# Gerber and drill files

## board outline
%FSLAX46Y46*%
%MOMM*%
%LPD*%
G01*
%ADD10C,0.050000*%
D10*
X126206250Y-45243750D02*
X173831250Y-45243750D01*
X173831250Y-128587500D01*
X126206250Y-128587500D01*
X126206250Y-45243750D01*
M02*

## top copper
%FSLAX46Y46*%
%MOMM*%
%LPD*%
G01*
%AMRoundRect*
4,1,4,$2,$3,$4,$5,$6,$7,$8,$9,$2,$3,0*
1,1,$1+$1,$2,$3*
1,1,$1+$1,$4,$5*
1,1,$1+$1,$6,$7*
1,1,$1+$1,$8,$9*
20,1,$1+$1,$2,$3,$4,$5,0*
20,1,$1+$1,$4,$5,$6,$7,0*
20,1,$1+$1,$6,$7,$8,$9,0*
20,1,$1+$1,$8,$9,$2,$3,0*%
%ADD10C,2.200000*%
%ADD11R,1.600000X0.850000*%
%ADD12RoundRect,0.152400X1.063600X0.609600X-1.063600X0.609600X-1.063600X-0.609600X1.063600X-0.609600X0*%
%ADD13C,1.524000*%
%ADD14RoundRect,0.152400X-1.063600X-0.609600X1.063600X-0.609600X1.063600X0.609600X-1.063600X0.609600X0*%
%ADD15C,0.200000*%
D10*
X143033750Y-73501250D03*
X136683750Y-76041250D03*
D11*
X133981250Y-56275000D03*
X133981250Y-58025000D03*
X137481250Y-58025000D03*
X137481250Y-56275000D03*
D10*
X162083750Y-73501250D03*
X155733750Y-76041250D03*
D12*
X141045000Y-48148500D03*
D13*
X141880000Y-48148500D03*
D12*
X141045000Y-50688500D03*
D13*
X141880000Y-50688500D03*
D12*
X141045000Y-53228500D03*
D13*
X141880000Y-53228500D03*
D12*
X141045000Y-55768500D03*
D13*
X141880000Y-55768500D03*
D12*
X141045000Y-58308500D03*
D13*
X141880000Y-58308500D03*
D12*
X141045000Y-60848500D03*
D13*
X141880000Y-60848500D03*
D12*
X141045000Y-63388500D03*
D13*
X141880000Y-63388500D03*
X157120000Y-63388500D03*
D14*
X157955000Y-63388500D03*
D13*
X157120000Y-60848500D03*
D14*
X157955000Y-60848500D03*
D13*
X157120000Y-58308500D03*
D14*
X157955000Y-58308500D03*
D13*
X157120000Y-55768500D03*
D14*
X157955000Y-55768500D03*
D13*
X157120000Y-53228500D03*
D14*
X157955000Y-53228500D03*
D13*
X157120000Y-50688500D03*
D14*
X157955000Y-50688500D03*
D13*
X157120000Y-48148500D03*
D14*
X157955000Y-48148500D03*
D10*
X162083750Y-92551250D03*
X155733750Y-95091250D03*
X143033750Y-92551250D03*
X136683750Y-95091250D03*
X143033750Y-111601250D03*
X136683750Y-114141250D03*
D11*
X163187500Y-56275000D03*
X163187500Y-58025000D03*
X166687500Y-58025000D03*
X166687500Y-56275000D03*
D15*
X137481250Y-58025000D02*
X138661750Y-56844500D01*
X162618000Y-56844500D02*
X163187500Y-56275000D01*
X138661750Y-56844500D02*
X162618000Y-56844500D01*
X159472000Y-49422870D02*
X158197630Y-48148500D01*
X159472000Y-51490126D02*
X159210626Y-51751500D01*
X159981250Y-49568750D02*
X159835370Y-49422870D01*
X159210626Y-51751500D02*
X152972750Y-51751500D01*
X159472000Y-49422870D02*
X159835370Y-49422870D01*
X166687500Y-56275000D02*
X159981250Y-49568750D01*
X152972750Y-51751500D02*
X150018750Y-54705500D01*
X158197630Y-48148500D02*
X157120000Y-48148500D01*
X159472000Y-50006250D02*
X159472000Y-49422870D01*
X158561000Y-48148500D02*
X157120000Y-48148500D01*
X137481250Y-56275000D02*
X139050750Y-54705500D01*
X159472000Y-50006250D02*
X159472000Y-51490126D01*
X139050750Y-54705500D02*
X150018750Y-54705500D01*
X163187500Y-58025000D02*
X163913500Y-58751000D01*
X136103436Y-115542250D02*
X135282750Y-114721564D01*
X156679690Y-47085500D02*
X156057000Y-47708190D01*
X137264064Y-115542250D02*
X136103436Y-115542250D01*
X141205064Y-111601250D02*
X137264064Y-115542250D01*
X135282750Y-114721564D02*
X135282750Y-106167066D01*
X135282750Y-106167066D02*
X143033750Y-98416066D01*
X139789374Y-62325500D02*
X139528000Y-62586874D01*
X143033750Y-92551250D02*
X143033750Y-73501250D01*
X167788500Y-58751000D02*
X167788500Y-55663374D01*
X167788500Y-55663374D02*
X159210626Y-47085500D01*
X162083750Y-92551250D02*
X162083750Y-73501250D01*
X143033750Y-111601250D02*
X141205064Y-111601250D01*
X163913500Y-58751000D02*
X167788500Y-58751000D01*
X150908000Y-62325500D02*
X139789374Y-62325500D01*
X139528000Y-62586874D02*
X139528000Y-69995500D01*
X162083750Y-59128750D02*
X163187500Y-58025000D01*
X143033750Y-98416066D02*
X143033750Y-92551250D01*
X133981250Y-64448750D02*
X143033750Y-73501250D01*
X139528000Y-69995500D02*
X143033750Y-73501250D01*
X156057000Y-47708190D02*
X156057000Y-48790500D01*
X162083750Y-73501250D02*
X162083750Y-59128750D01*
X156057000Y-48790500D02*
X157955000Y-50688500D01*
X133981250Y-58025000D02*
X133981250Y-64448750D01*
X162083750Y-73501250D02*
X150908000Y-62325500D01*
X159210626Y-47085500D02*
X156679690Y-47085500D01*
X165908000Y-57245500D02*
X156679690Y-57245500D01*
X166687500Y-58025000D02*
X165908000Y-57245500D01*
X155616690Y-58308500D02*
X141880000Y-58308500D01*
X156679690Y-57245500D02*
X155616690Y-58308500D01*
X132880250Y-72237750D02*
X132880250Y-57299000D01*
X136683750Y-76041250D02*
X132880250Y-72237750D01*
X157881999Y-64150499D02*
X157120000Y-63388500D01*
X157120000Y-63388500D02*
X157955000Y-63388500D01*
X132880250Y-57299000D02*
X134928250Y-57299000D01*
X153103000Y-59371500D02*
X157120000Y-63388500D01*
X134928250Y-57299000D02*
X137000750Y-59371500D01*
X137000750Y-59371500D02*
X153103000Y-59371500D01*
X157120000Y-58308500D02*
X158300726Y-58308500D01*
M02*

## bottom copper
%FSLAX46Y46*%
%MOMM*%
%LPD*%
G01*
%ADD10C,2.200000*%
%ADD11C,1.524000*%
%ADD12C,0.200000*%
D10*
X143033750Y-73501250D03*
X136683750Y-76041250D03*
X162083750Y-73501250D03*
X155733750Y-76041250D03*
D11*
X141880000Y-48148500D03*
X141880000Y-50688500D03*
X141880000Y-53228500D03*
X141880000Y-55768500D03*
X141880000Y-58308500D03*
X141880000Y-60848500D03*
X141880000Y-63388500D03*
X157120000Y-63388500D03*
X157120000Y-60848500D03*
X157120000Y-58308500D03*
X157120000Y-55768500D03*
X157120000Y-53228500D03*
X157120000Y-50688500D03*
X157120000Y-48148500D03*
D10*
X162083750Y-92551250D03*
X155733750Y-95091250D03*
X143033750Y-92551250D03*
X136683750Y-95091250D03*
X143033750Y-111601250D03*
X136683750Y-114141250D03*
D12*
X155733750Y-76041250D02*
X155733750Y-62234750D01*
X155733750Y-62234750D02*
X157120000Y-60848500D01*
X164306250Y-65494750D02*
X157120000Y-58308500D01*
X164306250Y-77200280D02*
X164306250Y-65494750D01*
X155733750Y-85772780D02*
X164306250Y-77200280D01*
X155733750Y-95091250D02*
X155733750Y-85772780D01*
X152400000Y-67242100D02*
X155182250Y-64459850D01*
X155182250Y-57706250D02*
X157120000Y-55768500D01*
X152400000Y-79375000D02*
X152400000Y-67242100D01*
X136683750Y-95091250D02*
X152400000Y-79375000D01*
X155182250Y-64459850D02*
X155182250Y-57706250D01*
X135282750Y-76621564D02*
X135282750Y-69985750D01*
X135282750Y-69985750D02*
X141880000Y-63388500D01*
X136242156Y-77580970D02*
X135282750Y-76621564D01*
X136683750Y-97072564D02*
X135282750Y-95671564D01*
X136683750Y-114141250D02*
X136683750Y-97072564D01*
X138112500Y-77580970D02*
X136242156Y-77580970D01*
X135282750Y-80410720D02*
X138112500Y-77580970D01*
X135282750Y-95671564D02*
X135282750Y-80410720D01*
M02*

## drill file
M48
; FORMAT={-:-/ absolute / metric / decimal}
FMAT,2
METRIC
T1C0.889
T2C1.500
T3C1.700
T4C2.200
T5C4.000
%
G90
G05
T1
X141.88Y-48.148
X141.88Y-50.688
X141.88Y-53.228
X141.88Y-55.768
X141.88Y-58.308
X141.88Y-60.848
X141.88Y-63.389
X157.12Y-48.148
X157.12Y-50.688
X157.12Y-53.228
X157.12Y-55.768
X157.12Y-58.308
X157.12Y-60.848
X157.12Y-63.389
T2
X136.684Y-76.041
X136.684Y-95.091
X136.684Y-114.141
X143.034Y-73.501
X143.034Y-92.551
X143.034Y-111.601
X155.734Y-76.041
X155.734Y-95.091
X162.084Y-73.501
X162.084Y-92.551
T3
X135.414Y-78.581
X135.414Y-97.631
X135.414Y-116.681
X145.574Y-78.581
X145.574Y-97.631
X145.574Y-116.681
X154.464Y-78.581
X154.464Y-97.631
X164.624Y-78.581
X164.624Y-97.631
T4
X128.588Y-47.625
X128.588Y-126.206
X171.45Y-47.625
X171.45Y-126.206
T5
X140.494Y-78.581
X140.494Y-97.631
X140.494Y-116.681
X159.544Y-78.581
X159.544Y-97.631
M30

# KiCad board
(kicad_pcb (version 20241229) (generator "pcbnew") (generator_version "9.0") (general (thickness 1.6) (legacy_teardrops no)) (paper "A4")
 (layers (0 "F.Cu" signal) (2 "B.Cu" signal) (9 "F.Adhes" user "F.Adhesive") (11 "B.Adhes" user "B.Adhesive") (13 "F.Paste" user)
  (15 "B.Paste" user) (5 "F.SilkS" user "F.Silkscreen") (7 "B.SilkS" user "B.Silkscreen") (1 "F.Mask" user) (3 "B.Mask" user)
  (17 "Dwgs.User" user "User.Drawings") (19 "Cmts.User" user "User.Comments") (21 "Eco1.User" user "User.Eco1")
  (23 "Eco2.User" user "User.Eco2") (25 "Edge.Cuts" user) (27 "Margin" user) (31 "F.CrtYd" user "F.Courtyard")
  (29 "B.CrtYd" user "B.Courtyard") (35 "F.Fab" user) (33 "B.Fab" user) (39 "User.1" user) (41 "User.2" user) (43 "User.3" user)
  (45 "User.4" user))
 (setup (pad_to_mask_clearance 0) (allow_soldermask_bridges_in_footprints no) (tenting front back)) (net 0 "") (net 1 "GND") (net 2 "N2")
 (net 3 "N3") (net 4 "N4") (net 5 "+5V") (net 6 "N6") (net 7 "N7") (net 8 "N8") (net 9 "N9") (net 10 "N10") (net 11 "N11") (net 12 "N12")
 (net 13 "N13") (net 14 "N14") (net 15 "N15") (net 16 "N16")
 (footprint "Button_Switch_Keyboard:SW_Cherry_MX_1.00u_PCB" (layer "F.Cu") (at 143.03375 73.50125)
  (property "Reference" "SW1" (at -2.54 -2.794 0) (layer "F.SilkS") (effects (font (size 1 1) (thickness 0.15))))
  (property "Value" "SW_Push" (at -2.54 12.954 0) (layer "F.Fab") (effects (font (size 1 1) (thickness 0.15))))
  (pad "" np_thru_hole circle (at -7.62 5.08) (size 1.7 1.7) (drill 1.7) (layers "*.Cu" "*.Mask"))
  (pad "" np_thru_hole circle (at -2.54 5.08) (size 4 4) (drill 4) (layers "*.Cu" "*.Mask"))
  (pad "" np_thru_hole circle (at 2.54 5.08) (size 1.7 1.7) (drill 1.7) (layers "*.Cu" "*.Mask"))
  (pad "1" thru_hole circle (at 0 0) (size 2.2 2.2) (drill 1.5) (layers "*.Cu" "*.Mask") (remove_unused_layers no) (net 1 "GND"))
  (pad "2" thru_hole circle (at -6.35 2.54) (size 2.2 2.2) (drill 1.5) (layers "*.Cu" "*.Mask") (remove_unused_layers no) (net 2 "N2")))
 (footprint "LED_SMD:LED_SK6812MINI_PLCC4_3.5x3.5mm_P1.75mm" (layer "F.Cu") (at 135.73125 57.15)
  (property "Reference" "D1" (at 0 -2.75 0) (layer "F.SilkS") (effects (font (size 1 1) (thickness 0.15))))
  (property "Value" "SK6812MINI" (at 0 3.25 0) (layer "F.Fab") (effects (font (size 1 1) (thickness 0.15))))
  (pad "1" smd rect (at -1.75 -0.875) (size 1.6 0.85) (layers "F.Cu" "F.Mask" "F.Paste") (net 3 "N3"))
  (pad "2" smd rect (at -1.75 0.875) (size 1.6 0.85) (layers "F.Cu" "F.Mask" "F.Paste") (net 1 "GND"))
  (pad "3" smd rect (at 1.75 0.875) (size 1.6 0.85) (layers "F.Cu" "F.Mask" "F.Paste") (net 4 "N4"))
  (pad "4" smd rect (at 1.75 -0.875) (size 1.6 0.85) (layers "F.Cu" "F.Mask" "F.Paste") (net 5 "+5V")))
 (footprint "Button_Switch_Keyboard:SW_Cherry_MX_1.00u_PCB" (layer "F.Cu") (at 162.08375 73.50125)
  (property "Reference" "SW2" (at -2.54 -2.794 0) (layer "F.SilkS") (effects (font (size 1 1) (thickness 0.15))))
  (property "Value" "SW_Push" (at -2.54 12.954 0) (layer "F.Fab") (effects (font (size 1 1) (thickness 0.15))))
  (pad "" np_thru_hole circle (at -7.62 5.08) (size 1.7 1.7) (drill 1.7) (layers "*.Cu" "*.Mask"))
  (pad "" np_thru_hole circle (at -2.54 5.08) (size 4 4) (drill 4) (layers "*.Cu" "*.Mask"))
  (pad "" np_thru_hole circle (at 2.54 5.08) (size 1.7 1.7) (drill 1.7) (layers "*.Cu" "*.Mask"))
  (pad "1" thru_hole circle (at 0 0) (size 2.2 2.2) (drill 1.5) (layers "*.Cu" "*.Mask") (remove_unused_layers no) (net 1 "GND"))
  (pad "2" thru_hole circle (at -6.35 2.54) (size 2.2 2.2) (drill 1.5) (layers "*.Cu" "*.Mask") (remove_unused_layers no) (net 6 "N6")))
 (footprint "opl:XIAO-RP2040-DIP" (layer "F.Cu") (at 149.5 55.7685)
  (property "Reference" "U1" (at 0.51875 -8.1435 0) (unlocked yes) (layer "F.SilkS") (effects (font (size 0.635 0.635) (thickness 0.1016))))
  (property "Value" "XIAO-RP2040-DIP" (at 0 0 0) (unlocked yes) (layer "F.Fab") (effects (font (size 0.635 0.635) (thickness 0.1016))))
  (pad "1" smd roundrect (at -8.455 -7.62 180) (size 2.432 1.524) (layers "F.Cu" "F.Mask") (roundrect_rratio 0.1) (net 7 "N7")
   (thermal_bridge_angle 45))
  (pad "1" thru_hole circle (at -7.62 -7.62 180) (size 1.524 1.524) (drill 0.889) (layers "*.Cu" "*.Mask") (remove_unused_layers no)
   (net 7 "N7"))
  (pad "2" smd roundrect (at -8.455 -5.08 180) (size 2.432 1.524) (layers "F.Cu" "F.Mask") (roundrect_rratio 0.1) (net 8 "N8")
   (thermal_bridge_angle 45))
  (pad "2" thru_hole circle (at -7.62 -5.08 180) (size 1.524 1.524) (drill 0.889) (layers "*.Cu" "*.Mask") (remove_unused_layers no)
   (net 8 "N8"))
  (pad "3" smd roundrect (at -8.455 -2.54 180) (size 2.432 1.524) (layers "F.Cu" "F.Mask") (roundrect_rratio 0.1) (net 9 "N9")
   (thermal_bridge_angle 45))
  (pad "3" thru_hole circle (at -7.62 -2.54 180) (size 1.524 1.524) (drill 0.889) (layers "*.Cu" "*.Mask") (remove_unused_layers no)
   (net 9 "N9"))
  (pad "4" smd roundrect (at -8.455 0 180) (size 2.432 1.524) (layers "F.Cu" "F.Mask") (roundrect_rratio 0.1) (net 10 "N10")
   (thermal_bridge_angle 45))
  (pad "4" thru_hole circle (at -7.62 0 180) (size 1.524 1.524) (drill 0.889) (layers "*.Cu" "*.Mask") (remove_unused_layers no)
   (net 10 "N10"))
  (pad "5" smd roundrect (at -8.455 2.54 180) (size 2.432 1.524) (layers "F.Cu" "F.Mask") (roundrect_rratio 0.1) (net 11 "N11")
   (thermal_bridge_angle 45))
  (pad "5" thru_hole circle (at -7.62 2.54 180) (size 1.524 1.524) (drill 0.889) (layers "*.Cu" "*.Mask") (remove_unused_layers no)
   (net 11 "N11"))
  (pad "6" smd roundrect (at -8.455 5.08 180) (size 2.432 1.524) (layers "F.Cu" "F.Mask") (roundrect_rratio 0.1) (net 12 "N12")
   (thermal_bridge_angle 45))
  (pad "6" thru_hole circle (at -7.62 5.08 180) (size 1.524 1.524) (drill 0.889) (layers "*.Cu" "*.Mask") (remove_unused_layers no)
   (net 12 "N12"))
  (pad "7" smd roundrect (at -8.455 7.62 180) (size 2.432 1.524) (layers "F.Cu" "F.Mask") (roundrect_rratio 0.1) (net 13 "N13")
   (thermal_bridge_angle 45))
  (pad "7" thru_hole circle (at -7.62 7.62 180) (size 1.524 1.524) (drill 0.889) (layers "*.Cu" "*.Mask") (remove_unused_layers no)
   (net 13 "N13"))
  (pad "8" thru_hole circle (at 7.62 7.62) (size 1.524 1.524) (drill 0.889) (layers "*.Cu" "*.Mask") (remove_unused_layers no) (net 2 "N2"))
  (pad "8" smd roundrect (at 8.455 7.62) (size 2.432 1.524) (layers "F.Cu" "F.Mask") (roundrect_rratio 0.1) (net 2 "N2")
   (thermal_bridge_angle 45))
  (pad "9" thru_hole circle (at 7.62 5.08) (size 1.524 1.524) (drill 0.889) (layers "*.Cu" "*.Mask") (remove_unused_layers no) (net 6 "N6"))
  (pad "9" smd roundrect (at 8.455 5.08) (size 2.432 1.524) (layers "F.Cu" "F.Mask") (roundrect_rratio 0.1) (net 6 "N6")
   (thermal_bridge_angle 45))
  (pad "10" thru_hole circle (at 7.62 2.54) (size 1.524 1.524) (drill 0.889) (layers "*.Cu" "*.Mask") (remove_unused_layers no)
   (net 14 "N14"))
  (pad "10" smd roundrect (at 8.455 2.54) (size 2.432 1.524) (layers "F.Cu" "F.Mask") (roundrect_rratio 0.1) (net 14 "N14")
   (thermal_bridge_angle 45))
  (pad "11" thru_hole circle (at 7.62 0) (size 1.524 1.524) (drill 0.889) (layers "*.Cu" "*.Mask") (remove_unused_layers no) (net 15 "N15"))
  (pad "11" smd roundrect (at 8.455 0) (size 2.432 1.524) (layers "F.Cu" "F.Mask") (roundrect_rratio 0.1) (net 15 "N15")
   (thermal_bridge_angle 45))
  (pad "12" thru_hole circle (at 7.62 -2.54) (size 1.524 1.524) (drill 0.889) (layers "*.Cu" "*.Mask") (remove_unused_layers no)
   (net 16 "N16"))
  (pad "12" smd roundrect (at 8.455 -2.54) (size 2.432 1.524) (layers "F.Cu" "F.Mask") (roundrect_rratio 0.1) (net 16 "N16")
   (thermal_bridge_angle 45))
  (pad "13" thru_hole circle (at 7.62 -5.08) (size 1.524 1.524) (drill 0.889) (layers "*.Cu" "*.Mask") (remove_unused_layers no)
   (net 1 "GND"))
  (pad "13" smd roundrect (at 8.455 -5.08) (size 2.432 1.524) (layers "F.Cu" "F.Mask") (roundrect_rratio 0.1) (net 1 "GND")
   (thermal_bridge_angle 45))
  (pad "14" thru_hole circle (at 7.62 -7.62) (size 1.524 1.524) (drill 0.889) (layers "*.Cu" "*.Mask") (remove_unused_layers no)
   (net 5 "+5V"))
  (pad "14" smd roundrect (at 8.455 -7.62) (size 2.432 1.524) (layers "F.Cu" "F.Mask") (roundrect_rratio 0.1) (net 5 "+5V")
   (thermal_bridge_angle 45)))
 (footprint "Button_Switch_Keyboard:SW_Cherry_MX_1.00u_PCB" (layer "F.Cu") (at 162.08375 92.55125)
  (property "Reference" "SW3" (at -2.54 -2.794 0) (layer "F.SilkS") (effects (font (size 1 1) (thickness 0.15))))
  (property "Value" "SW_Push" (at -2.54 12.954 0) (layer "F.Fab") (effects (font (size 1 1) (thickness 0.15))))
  (pad "" np_thru_hole circle (at -7.62 5.08) (size 1.7 1.7) (drill 1.7) (layers "*.Cu" "*.Mask"))
  (pad "" np_thru_hole circle (at -2.54 5.08) (size 4 4) (drill 4) (layers "*.Cu" "*.Mask"))
  (pad "" np_thru_hole circle (at 2.54 5.08) (size 1.7 1.7) (drill 1.7) (layers "*.Cu" "*.Mask"))
  (pad "1" thru_hole circle (at 0 0) (size 2.2 2.2) (drill 1.5) (layers "*.Cu" "*.Mask") (remove_unused_layers no) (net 1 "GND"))
  (pad "2" thru_hole circle (at -6.35 2.54) (size 2.2 2.2) (drill 1.5) (layers "*.Cu" "*.Mask") (remove_unused_layers no) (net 14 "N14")))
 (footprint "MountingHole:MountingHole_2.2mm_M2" (layer "F.Cu") (at 171.45 47.625)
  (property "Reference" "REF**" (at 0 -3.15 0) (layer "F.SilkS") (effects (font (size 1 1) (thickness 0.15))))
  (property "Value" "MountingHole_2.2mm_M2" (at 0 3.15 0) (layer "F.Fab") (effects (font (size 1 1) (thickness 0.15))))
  (pad "" np_thru_hole circle (at 0 0) (size 2.2 2.2) (drill 2.2) (layers "*.Cu" "*.Mask")))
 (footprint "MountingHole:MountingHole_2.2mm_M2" (layer "F.Cu") (at 128.5875 47.625)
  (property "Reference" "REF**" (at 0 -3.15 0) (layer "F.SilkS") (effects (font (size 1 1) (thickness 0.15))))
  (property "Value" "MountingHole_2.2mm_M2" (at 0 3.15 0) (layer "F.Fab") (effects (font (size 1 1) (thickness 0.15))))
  (pad "" np_thru_hole circle (at 0 0) (size 2.2 2.2) (drill 2.2) (layers "*.Cu" "*.Mask")))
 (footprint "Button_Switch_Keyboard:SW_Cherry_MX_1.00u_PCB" (layer "F.Cu") (at 143.03375 92.55125)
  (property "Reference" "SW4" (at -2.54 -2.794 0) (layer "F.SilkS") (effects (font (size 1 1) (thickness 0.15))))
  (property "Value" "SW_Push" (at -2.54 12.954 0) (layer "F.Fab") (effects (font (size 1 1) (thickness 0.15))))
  (pad "" np_thru_hole circle (at -7.62 5.08) (size 1.7 1.7) (drill 1.7) (layers "*.Cu" "*.Mask"))
  (pad "" np_thru_hole circle (at -2.54 5.08) (size 4 4) (drill 4) (layers "*.Cu" "*.Mask"))
  (pad "" np_thru_hole circle (at 2.54 5.08) (size 1.7 1.7) (drill 1.7) (layers "*.Cu" "*.Mask"))
  (pad "1" thru_hole circle (at 0 0) (size 2.2 2.2) (drill 1.5) (layers "*.Cu" "*.Mask") (remove_unused_layers no) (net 1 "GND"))
  (pad "2" thru_hole circle (at -6.35 2.54) (size 2.2 2.2) (drill 1.5) (layers "*.Cu" "*.Mask") (remove_unused_layers no) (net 15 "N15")))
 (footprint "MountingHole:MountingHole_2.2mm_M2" (layer "F.Cu") (at 171.45 126.20625)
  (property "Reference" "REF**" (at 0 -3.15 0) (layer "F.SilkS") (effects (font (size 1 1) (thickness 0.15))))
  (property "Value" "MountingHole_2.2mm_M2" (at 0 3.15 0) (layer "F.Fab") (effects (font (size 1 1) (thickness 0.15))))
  (pad "" np_thru_hole circle (at 0 0) (size 2.2 2.2) (drill 2.2) (layers "*.Cu" "*.Mask")))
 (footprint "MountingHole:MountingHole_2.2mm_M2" (layer "F.Cu") (at 128.5875 126.20625)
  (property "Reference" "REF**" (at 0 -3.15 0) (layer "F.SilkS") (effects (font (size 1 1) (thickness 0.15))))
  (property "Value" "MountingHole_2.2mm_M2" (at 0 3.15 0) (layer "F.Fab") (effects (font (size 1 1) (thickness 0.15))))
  (pad "" np_thru_hole circle (at 0 0) (size 2.2 2.2) (drill 2.2) (layers "*.Cu" "*.Mask")))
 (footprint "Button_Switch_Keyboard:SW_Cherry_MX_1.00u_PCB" (layer "F.Cu") (at 143.03375 111.60125)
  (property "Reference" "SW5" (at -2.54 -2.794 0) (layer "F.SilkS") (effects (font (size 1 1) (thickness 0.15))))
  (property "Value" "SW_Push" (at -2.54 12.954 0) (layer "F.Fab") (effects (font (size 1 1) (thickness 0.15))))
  (pad "" np_thru_hole circle (at -7.62 5.08) (size 1.7 1.7) (drill 1.7) (layers "*.Cu" "*.Mask"))
  (pad "" np_thru_hole circle (at -2.54 5.08) (size 4 4) (drill 4) (layers "*.Cu" "*.Mask"))
  (pad "" np_thru_hole circle (at 2.54 5.08) (size 1.7 1.7) (drill 1.7) (layers "*.Cu" "*.Mask"))
  (pad "1" thru_hole circle (at 0 0) (size 2.2 2.2) (drill 1.5) (layers "*.Cu" "*.Mask") (remove_unused_layers no) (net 1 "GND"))
  (pad "2" thru_hole circle (at -6.35 2.54) (size 2.2 2.2) (drill 1.5) (layers "*.Cu" "*.Mask") (remove_unused_layers no) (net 13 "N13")))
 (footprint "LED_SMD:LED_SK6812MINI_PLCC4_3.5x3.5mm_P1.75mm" (layer "F.Cu") (at 164.9375 57.15)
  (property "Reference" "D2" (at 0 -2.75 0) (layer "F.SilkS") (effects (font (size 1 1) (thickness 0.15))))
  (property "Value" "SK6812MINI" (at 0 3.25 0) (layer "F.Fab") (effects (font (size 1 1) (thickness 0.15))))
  (pad "1" smd rect (at -1.75 -0.875) (size 1.6 0.85) (layers "F.Cu" "F.Mask" "F.Paste") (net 4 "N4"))
  (pad "2" smd rect (at -1.75 0.875) (size 1.6 0.85) (layers "F.Cu" "F.Mask" "F.Paste") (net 1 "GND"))
  (pad "3" smd rect (at 1.75 0.875) (size 1.6 0.85) (layers "F.Cu" "F.Mask" "F.Paste") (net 11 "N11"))
  (pad "4" smd rect (at 1.75 -0.875) (size 1.6 0.85) (layers "F.Cu" "F.Mask" "F.Paste") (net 5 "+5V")))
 (gr_rect (start 126.20625 45.24375) (end 173.83125 128.5875) (stroke (width 0.05) (type default)) (fill no) (layer "Edge.Cuts"))
 (segment (start 137.48125 58.025) (end 138.66175 56.8445) (width 0.2) (layer "F.Cu") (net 4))
 (segment (start 162.618 56.8445) (end 163.1875 56.275) (width 0.2) (layer "F.Cu") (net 4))
 (segment (start 138.66175 56.8445) (end 162.618 56.8445) (width 0.2) (layer "F.Cu") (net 4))
 (segment (start 159.472 49.42287) (end 158.19763 48.1485) (width 0.2) (layer "F.Cu") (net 5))
 (segment (start 159.472 51.490126) (end 159.210626 51.7515) (width 0.2) (layer "F.Cu") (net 5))
 (segment (start 159.98125 49.56875) (end 159.83537 49.42287) (width 0.2) (layer "F.Cu") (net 5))
 (segment (start 159.210626 51.7515) (end 152.97275 51.7515) (width 0.2) (layer "F.Cu") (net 5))
 (segment (start 159.472 49.42287) (end 159.83537 49.42287) (width 0.2) (layer "F.Cu") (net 5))
 (segment (start 166.6875 56.275) (end 159.98125 49.56875) (width 0.2) (layer "F.Cu") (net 5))
 (segment (start 152.97275 51.7515) (end 150.01875 54.7055) (width 0.2) (layer "F.Cu") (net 5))
 (segment (start 158.19763 48.1485) (end 157.12 48.1485) (width 0.2) (layer "F.Cu") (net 5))
 (segment (start 159.472 50.00625) (end 159.472 49.42287) (width 0.2) (layer "F.Cu") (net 5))
 (segment (start 158.561 48.1485) (end 157.12 48.1485) (width 0.2) (layer "F.Cu") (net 5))
 (segment (start 137.48125 56.275) (end 139.05075 54.7055) (width 0.2) (layer "F.Cu") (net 5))
 (segment (start 159.472 50.00625) (end 159.472 51.490126) (width 0.2) (layer "F.Cu") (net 5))
 (segment (start 139.05075 54.7055) (end 150.01875 54.7055) (width 0.2) (layer "F.Cu") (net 5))
 (segment (start 163.1875 58.025) (end 163.9135 58.751) (width 0.2) (layer "F.Cu") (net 1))
 (segment (start 136.103436 115.54225) (end 135.28275 114.721564) (width 0.2) (layer "F.Cu") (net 1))
 (segment (start 156.67969 47.0855) (end 156.057 47.70819) (width 0.2) (layer "F.Cu") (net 1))
 (segment (start 137.264064 115.54225) (end 136.103436 115.54225) (width 0.2) (layer "F.Cu") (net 1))
 (segment (start 141.205064 111.60125) (end 137.264064 115.54225) (width 0.2) (layer "F.Cu") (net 1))
 (segment (start 135.28275 114.721564) (end 135.28275 106.167066) (width 0.2) (layer "F.Cu") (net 1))
 (segment (start 135.28275 106.167066) (end 143.03375 98.416066) (width 0.2) (layer "F.Cu") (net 1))
 (segment (start 139.789374 62.3255) (end 139.528 62.586874) (width 0.2) (layer "F.Cu") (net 1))
 (segment (start 143.03375 92.55125) (end 143.03375 73.50125) (width 0.2) (layer "F.Cu") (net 1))
 (segment (start 167.7885 58.751) (end 167.7885 55.663374) (width 0.2) (layer "F.Cu") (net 1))
 (segment (start 167.7885 55.663374) (end 159.210626 47.0855) (width 0.2) (layer "F.Cu") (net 1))
 (segment (start 162.08375 92.55125) (end 162.08375 73.50125) (width 0.2) (layer "F.Cu") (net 1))
 (segment (start 143.03375 111.60125) (end 141.205064 111.60125) (width 0.2) (layer "F.Cu") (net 1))
 (segment (start 163.9135 58.751) (end 167.7885 58.751) (width 0.2) (layer "F.Cu") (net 1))
 (segment (start 150.908 62.3255) (end 139.789374 62.3255) (width 0.2) (layer "F.Cu") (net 1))
 (segment (start 139.528 62.586874) (end 139.528 69.9955) (width 0.2) (layer "F.Cu") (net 1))
 (segment (start 162.08375 59.12875) (end 163.1875 58.025) (width 0.2) (layer "F.Cu") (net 1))
 (segment (start 143.03375 98.416066) (end 143.03375 92.55125) (width 0.2) (layer "F.Cu") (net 1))
 (segment (start 133.98125 64.44875) (end 143.03375 73.50125) (width 0.2) (layer "F.Cu") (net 1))
 (segment (start 139.528 69.9955) (end 143.03375 73.50125) (width 0.2) (layer "F.Cu") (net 1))
 (segment (start 156.057 47.70819) (end 156.057 48.7905) (width 0.2) (layer "F.Cu") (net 1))
 (segment (start 162.08375 73.50125) (end 162.08375 59.12875) (width 0.2) (layer "F.Cu") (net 1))
 (segment (start 156.057 48.7905) (end 157.955 50.6885) (width 0.2) (layer "F.Cu") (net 1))
 (segment (start 133.98125 58.025) (end 133.98125 64.44875) (width 0.2) (layer "F.Cu") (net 1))
 (segment (start 162.08375 73.50125) (end 150.908 62.3255) (width 0.2) (layer "F.Cu") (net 1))
 (segment (start 159.210626 47.0855) (end 156.67969 47.0855) (width 0.2) (layer "F.Cu") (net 1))
 (segment (start 165.908 57.2455) (end 156.67969 57.2455) (width 0.2) (layer "F.Cu") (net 11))
 (segment (start 166.6875 58.025) (end 165.908 57.2455) (width 0.2) (layer "F.Cu") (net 11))
 (segment (start 155.61669 58.3085) (end 141.88 58.3085) (width 0.2) (layer "F.Cu") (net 11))
 (segment (start 156.67969 57.2455) (end 155.61669 58.3085) (width 0.2) (layer "F.Cu") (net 11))
 (segment (start 132.88025 72.23775) (end 132.88025 57.299) (width 0.2) (layer "F.Cu") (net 2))
 (segment (start 136.68375 76.04125) (end 132.88025 72.23775) (width 0.2) (layer "F.Cu") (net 2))
 (segment (start 157.881999 64.150499) (end 157.12 63.3885) (width 0.2) (layer "F.Cu") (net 2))
 (segment (start 157.12 63.3885) (end 157.955 63.3885) (width 0.2) (layer "F.Cu") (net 2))
 (segment (start 132.88025 57.299) (end 134.92825 57.299) (width 0.2) (layer "F.Cu") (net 2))
 (segment (start 153.103 59.3715) (end 157.12 63.3885) (width 0.2) (layer "F.Cu") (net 2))
 (segment (start 134.92825 57.299) (end 137.00075 59.3715) (width 0.2) (layer "F.Cu") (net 2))
 (segment (start 137.00075 59.3715) (end 153.103 59.3715) (width 0.2) (layer "F.Cu") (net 2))
 (segment (start 155.73375 76.04125) (end 155.73375 62.23475) (width 0.2) (layer "B.Cu") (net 6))
 (segment (start 155.73375 62.23475) (end 157.12 60.8485) (width 0.2) (layer "B.Cu") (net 6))
 (segment (start 157.12 58.3085) (end 158.300726 58.3085) (width 0.2) (layer "F.Cu") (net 14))
 (segment (start 164.30625 65.49475) (end 157.12 58.3085) (width 0.2) (layer "B.Cu") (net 14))
 (segment (start 164.30625 77.20028) (end 164.30625 65.49475) (width 0.2) (layer "B.Cu") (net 14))
 (segment (start 155.73375 85.77278) (end 164.30625 77.20028) (width 0.2) (layer "B.Cu") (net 14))
 (segment (start 155.73375 95.09125) (end 155.73375 85.77278) (width 0.2) (layer "B.Cu") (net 14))
 (segment (start 152.4 67.2421) (end 155.18225 64.45985) (width 0.2) (layer "B.Cu") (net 15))
 (segment (start 155.18225 57.70625) (end 157.12 55.7685) (width 0.2) (layer "B.Cu") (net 15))
 (segment (start 152.4 79.375) (end 152.4 67.2421) (width 0.2) (layer "B.Cu") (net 15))
 (segment (start 136.68375 95.09125) (end 152.4 79.375) (width 0.2) (layer "B.Cu") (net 15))
 (segment (start 155.18225 64.45985) (end 155.18225 57.70625) (width 0.2) (layer "B.Cu") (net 15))
 (segment (start 135.28275 76.621564) (end 135.28275 69.98575) (width 0.2) (layer "B.Cu") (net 13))
 (segment (start 135.28275 69.98575) (end 141.88 63.3885) (width 0.2) (layer "B.Cu") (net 13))
 (segment (start 136.242156 77.58097) (end 135.28275 76.621564) (width 0.2) (layer "B.Cu") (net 13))
 (segment (start 136.68375 97.072564) (end 135.28275 95.671564) (width 0.2) (layer "B.Cu") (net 13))
 (segment (start 136.68375 114.14125) (end 136.68375 97.072564) (width 0.2) (layer "B.Cu") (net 13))
 (segment (start 138.1125 77.58097) (end 136.242156 77.58097) (width 0.2) (layer "B.Cu") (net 13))
 (segment (start 135.28275 80.41072) (end 138.1125 77.58097) (width 0.2) (layer "B.Cu") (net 13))
 (segment (start 135.28275 95.671564) (end 135.28275 80.41072) (width 0.2) (layer "B.Cu") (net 13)))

